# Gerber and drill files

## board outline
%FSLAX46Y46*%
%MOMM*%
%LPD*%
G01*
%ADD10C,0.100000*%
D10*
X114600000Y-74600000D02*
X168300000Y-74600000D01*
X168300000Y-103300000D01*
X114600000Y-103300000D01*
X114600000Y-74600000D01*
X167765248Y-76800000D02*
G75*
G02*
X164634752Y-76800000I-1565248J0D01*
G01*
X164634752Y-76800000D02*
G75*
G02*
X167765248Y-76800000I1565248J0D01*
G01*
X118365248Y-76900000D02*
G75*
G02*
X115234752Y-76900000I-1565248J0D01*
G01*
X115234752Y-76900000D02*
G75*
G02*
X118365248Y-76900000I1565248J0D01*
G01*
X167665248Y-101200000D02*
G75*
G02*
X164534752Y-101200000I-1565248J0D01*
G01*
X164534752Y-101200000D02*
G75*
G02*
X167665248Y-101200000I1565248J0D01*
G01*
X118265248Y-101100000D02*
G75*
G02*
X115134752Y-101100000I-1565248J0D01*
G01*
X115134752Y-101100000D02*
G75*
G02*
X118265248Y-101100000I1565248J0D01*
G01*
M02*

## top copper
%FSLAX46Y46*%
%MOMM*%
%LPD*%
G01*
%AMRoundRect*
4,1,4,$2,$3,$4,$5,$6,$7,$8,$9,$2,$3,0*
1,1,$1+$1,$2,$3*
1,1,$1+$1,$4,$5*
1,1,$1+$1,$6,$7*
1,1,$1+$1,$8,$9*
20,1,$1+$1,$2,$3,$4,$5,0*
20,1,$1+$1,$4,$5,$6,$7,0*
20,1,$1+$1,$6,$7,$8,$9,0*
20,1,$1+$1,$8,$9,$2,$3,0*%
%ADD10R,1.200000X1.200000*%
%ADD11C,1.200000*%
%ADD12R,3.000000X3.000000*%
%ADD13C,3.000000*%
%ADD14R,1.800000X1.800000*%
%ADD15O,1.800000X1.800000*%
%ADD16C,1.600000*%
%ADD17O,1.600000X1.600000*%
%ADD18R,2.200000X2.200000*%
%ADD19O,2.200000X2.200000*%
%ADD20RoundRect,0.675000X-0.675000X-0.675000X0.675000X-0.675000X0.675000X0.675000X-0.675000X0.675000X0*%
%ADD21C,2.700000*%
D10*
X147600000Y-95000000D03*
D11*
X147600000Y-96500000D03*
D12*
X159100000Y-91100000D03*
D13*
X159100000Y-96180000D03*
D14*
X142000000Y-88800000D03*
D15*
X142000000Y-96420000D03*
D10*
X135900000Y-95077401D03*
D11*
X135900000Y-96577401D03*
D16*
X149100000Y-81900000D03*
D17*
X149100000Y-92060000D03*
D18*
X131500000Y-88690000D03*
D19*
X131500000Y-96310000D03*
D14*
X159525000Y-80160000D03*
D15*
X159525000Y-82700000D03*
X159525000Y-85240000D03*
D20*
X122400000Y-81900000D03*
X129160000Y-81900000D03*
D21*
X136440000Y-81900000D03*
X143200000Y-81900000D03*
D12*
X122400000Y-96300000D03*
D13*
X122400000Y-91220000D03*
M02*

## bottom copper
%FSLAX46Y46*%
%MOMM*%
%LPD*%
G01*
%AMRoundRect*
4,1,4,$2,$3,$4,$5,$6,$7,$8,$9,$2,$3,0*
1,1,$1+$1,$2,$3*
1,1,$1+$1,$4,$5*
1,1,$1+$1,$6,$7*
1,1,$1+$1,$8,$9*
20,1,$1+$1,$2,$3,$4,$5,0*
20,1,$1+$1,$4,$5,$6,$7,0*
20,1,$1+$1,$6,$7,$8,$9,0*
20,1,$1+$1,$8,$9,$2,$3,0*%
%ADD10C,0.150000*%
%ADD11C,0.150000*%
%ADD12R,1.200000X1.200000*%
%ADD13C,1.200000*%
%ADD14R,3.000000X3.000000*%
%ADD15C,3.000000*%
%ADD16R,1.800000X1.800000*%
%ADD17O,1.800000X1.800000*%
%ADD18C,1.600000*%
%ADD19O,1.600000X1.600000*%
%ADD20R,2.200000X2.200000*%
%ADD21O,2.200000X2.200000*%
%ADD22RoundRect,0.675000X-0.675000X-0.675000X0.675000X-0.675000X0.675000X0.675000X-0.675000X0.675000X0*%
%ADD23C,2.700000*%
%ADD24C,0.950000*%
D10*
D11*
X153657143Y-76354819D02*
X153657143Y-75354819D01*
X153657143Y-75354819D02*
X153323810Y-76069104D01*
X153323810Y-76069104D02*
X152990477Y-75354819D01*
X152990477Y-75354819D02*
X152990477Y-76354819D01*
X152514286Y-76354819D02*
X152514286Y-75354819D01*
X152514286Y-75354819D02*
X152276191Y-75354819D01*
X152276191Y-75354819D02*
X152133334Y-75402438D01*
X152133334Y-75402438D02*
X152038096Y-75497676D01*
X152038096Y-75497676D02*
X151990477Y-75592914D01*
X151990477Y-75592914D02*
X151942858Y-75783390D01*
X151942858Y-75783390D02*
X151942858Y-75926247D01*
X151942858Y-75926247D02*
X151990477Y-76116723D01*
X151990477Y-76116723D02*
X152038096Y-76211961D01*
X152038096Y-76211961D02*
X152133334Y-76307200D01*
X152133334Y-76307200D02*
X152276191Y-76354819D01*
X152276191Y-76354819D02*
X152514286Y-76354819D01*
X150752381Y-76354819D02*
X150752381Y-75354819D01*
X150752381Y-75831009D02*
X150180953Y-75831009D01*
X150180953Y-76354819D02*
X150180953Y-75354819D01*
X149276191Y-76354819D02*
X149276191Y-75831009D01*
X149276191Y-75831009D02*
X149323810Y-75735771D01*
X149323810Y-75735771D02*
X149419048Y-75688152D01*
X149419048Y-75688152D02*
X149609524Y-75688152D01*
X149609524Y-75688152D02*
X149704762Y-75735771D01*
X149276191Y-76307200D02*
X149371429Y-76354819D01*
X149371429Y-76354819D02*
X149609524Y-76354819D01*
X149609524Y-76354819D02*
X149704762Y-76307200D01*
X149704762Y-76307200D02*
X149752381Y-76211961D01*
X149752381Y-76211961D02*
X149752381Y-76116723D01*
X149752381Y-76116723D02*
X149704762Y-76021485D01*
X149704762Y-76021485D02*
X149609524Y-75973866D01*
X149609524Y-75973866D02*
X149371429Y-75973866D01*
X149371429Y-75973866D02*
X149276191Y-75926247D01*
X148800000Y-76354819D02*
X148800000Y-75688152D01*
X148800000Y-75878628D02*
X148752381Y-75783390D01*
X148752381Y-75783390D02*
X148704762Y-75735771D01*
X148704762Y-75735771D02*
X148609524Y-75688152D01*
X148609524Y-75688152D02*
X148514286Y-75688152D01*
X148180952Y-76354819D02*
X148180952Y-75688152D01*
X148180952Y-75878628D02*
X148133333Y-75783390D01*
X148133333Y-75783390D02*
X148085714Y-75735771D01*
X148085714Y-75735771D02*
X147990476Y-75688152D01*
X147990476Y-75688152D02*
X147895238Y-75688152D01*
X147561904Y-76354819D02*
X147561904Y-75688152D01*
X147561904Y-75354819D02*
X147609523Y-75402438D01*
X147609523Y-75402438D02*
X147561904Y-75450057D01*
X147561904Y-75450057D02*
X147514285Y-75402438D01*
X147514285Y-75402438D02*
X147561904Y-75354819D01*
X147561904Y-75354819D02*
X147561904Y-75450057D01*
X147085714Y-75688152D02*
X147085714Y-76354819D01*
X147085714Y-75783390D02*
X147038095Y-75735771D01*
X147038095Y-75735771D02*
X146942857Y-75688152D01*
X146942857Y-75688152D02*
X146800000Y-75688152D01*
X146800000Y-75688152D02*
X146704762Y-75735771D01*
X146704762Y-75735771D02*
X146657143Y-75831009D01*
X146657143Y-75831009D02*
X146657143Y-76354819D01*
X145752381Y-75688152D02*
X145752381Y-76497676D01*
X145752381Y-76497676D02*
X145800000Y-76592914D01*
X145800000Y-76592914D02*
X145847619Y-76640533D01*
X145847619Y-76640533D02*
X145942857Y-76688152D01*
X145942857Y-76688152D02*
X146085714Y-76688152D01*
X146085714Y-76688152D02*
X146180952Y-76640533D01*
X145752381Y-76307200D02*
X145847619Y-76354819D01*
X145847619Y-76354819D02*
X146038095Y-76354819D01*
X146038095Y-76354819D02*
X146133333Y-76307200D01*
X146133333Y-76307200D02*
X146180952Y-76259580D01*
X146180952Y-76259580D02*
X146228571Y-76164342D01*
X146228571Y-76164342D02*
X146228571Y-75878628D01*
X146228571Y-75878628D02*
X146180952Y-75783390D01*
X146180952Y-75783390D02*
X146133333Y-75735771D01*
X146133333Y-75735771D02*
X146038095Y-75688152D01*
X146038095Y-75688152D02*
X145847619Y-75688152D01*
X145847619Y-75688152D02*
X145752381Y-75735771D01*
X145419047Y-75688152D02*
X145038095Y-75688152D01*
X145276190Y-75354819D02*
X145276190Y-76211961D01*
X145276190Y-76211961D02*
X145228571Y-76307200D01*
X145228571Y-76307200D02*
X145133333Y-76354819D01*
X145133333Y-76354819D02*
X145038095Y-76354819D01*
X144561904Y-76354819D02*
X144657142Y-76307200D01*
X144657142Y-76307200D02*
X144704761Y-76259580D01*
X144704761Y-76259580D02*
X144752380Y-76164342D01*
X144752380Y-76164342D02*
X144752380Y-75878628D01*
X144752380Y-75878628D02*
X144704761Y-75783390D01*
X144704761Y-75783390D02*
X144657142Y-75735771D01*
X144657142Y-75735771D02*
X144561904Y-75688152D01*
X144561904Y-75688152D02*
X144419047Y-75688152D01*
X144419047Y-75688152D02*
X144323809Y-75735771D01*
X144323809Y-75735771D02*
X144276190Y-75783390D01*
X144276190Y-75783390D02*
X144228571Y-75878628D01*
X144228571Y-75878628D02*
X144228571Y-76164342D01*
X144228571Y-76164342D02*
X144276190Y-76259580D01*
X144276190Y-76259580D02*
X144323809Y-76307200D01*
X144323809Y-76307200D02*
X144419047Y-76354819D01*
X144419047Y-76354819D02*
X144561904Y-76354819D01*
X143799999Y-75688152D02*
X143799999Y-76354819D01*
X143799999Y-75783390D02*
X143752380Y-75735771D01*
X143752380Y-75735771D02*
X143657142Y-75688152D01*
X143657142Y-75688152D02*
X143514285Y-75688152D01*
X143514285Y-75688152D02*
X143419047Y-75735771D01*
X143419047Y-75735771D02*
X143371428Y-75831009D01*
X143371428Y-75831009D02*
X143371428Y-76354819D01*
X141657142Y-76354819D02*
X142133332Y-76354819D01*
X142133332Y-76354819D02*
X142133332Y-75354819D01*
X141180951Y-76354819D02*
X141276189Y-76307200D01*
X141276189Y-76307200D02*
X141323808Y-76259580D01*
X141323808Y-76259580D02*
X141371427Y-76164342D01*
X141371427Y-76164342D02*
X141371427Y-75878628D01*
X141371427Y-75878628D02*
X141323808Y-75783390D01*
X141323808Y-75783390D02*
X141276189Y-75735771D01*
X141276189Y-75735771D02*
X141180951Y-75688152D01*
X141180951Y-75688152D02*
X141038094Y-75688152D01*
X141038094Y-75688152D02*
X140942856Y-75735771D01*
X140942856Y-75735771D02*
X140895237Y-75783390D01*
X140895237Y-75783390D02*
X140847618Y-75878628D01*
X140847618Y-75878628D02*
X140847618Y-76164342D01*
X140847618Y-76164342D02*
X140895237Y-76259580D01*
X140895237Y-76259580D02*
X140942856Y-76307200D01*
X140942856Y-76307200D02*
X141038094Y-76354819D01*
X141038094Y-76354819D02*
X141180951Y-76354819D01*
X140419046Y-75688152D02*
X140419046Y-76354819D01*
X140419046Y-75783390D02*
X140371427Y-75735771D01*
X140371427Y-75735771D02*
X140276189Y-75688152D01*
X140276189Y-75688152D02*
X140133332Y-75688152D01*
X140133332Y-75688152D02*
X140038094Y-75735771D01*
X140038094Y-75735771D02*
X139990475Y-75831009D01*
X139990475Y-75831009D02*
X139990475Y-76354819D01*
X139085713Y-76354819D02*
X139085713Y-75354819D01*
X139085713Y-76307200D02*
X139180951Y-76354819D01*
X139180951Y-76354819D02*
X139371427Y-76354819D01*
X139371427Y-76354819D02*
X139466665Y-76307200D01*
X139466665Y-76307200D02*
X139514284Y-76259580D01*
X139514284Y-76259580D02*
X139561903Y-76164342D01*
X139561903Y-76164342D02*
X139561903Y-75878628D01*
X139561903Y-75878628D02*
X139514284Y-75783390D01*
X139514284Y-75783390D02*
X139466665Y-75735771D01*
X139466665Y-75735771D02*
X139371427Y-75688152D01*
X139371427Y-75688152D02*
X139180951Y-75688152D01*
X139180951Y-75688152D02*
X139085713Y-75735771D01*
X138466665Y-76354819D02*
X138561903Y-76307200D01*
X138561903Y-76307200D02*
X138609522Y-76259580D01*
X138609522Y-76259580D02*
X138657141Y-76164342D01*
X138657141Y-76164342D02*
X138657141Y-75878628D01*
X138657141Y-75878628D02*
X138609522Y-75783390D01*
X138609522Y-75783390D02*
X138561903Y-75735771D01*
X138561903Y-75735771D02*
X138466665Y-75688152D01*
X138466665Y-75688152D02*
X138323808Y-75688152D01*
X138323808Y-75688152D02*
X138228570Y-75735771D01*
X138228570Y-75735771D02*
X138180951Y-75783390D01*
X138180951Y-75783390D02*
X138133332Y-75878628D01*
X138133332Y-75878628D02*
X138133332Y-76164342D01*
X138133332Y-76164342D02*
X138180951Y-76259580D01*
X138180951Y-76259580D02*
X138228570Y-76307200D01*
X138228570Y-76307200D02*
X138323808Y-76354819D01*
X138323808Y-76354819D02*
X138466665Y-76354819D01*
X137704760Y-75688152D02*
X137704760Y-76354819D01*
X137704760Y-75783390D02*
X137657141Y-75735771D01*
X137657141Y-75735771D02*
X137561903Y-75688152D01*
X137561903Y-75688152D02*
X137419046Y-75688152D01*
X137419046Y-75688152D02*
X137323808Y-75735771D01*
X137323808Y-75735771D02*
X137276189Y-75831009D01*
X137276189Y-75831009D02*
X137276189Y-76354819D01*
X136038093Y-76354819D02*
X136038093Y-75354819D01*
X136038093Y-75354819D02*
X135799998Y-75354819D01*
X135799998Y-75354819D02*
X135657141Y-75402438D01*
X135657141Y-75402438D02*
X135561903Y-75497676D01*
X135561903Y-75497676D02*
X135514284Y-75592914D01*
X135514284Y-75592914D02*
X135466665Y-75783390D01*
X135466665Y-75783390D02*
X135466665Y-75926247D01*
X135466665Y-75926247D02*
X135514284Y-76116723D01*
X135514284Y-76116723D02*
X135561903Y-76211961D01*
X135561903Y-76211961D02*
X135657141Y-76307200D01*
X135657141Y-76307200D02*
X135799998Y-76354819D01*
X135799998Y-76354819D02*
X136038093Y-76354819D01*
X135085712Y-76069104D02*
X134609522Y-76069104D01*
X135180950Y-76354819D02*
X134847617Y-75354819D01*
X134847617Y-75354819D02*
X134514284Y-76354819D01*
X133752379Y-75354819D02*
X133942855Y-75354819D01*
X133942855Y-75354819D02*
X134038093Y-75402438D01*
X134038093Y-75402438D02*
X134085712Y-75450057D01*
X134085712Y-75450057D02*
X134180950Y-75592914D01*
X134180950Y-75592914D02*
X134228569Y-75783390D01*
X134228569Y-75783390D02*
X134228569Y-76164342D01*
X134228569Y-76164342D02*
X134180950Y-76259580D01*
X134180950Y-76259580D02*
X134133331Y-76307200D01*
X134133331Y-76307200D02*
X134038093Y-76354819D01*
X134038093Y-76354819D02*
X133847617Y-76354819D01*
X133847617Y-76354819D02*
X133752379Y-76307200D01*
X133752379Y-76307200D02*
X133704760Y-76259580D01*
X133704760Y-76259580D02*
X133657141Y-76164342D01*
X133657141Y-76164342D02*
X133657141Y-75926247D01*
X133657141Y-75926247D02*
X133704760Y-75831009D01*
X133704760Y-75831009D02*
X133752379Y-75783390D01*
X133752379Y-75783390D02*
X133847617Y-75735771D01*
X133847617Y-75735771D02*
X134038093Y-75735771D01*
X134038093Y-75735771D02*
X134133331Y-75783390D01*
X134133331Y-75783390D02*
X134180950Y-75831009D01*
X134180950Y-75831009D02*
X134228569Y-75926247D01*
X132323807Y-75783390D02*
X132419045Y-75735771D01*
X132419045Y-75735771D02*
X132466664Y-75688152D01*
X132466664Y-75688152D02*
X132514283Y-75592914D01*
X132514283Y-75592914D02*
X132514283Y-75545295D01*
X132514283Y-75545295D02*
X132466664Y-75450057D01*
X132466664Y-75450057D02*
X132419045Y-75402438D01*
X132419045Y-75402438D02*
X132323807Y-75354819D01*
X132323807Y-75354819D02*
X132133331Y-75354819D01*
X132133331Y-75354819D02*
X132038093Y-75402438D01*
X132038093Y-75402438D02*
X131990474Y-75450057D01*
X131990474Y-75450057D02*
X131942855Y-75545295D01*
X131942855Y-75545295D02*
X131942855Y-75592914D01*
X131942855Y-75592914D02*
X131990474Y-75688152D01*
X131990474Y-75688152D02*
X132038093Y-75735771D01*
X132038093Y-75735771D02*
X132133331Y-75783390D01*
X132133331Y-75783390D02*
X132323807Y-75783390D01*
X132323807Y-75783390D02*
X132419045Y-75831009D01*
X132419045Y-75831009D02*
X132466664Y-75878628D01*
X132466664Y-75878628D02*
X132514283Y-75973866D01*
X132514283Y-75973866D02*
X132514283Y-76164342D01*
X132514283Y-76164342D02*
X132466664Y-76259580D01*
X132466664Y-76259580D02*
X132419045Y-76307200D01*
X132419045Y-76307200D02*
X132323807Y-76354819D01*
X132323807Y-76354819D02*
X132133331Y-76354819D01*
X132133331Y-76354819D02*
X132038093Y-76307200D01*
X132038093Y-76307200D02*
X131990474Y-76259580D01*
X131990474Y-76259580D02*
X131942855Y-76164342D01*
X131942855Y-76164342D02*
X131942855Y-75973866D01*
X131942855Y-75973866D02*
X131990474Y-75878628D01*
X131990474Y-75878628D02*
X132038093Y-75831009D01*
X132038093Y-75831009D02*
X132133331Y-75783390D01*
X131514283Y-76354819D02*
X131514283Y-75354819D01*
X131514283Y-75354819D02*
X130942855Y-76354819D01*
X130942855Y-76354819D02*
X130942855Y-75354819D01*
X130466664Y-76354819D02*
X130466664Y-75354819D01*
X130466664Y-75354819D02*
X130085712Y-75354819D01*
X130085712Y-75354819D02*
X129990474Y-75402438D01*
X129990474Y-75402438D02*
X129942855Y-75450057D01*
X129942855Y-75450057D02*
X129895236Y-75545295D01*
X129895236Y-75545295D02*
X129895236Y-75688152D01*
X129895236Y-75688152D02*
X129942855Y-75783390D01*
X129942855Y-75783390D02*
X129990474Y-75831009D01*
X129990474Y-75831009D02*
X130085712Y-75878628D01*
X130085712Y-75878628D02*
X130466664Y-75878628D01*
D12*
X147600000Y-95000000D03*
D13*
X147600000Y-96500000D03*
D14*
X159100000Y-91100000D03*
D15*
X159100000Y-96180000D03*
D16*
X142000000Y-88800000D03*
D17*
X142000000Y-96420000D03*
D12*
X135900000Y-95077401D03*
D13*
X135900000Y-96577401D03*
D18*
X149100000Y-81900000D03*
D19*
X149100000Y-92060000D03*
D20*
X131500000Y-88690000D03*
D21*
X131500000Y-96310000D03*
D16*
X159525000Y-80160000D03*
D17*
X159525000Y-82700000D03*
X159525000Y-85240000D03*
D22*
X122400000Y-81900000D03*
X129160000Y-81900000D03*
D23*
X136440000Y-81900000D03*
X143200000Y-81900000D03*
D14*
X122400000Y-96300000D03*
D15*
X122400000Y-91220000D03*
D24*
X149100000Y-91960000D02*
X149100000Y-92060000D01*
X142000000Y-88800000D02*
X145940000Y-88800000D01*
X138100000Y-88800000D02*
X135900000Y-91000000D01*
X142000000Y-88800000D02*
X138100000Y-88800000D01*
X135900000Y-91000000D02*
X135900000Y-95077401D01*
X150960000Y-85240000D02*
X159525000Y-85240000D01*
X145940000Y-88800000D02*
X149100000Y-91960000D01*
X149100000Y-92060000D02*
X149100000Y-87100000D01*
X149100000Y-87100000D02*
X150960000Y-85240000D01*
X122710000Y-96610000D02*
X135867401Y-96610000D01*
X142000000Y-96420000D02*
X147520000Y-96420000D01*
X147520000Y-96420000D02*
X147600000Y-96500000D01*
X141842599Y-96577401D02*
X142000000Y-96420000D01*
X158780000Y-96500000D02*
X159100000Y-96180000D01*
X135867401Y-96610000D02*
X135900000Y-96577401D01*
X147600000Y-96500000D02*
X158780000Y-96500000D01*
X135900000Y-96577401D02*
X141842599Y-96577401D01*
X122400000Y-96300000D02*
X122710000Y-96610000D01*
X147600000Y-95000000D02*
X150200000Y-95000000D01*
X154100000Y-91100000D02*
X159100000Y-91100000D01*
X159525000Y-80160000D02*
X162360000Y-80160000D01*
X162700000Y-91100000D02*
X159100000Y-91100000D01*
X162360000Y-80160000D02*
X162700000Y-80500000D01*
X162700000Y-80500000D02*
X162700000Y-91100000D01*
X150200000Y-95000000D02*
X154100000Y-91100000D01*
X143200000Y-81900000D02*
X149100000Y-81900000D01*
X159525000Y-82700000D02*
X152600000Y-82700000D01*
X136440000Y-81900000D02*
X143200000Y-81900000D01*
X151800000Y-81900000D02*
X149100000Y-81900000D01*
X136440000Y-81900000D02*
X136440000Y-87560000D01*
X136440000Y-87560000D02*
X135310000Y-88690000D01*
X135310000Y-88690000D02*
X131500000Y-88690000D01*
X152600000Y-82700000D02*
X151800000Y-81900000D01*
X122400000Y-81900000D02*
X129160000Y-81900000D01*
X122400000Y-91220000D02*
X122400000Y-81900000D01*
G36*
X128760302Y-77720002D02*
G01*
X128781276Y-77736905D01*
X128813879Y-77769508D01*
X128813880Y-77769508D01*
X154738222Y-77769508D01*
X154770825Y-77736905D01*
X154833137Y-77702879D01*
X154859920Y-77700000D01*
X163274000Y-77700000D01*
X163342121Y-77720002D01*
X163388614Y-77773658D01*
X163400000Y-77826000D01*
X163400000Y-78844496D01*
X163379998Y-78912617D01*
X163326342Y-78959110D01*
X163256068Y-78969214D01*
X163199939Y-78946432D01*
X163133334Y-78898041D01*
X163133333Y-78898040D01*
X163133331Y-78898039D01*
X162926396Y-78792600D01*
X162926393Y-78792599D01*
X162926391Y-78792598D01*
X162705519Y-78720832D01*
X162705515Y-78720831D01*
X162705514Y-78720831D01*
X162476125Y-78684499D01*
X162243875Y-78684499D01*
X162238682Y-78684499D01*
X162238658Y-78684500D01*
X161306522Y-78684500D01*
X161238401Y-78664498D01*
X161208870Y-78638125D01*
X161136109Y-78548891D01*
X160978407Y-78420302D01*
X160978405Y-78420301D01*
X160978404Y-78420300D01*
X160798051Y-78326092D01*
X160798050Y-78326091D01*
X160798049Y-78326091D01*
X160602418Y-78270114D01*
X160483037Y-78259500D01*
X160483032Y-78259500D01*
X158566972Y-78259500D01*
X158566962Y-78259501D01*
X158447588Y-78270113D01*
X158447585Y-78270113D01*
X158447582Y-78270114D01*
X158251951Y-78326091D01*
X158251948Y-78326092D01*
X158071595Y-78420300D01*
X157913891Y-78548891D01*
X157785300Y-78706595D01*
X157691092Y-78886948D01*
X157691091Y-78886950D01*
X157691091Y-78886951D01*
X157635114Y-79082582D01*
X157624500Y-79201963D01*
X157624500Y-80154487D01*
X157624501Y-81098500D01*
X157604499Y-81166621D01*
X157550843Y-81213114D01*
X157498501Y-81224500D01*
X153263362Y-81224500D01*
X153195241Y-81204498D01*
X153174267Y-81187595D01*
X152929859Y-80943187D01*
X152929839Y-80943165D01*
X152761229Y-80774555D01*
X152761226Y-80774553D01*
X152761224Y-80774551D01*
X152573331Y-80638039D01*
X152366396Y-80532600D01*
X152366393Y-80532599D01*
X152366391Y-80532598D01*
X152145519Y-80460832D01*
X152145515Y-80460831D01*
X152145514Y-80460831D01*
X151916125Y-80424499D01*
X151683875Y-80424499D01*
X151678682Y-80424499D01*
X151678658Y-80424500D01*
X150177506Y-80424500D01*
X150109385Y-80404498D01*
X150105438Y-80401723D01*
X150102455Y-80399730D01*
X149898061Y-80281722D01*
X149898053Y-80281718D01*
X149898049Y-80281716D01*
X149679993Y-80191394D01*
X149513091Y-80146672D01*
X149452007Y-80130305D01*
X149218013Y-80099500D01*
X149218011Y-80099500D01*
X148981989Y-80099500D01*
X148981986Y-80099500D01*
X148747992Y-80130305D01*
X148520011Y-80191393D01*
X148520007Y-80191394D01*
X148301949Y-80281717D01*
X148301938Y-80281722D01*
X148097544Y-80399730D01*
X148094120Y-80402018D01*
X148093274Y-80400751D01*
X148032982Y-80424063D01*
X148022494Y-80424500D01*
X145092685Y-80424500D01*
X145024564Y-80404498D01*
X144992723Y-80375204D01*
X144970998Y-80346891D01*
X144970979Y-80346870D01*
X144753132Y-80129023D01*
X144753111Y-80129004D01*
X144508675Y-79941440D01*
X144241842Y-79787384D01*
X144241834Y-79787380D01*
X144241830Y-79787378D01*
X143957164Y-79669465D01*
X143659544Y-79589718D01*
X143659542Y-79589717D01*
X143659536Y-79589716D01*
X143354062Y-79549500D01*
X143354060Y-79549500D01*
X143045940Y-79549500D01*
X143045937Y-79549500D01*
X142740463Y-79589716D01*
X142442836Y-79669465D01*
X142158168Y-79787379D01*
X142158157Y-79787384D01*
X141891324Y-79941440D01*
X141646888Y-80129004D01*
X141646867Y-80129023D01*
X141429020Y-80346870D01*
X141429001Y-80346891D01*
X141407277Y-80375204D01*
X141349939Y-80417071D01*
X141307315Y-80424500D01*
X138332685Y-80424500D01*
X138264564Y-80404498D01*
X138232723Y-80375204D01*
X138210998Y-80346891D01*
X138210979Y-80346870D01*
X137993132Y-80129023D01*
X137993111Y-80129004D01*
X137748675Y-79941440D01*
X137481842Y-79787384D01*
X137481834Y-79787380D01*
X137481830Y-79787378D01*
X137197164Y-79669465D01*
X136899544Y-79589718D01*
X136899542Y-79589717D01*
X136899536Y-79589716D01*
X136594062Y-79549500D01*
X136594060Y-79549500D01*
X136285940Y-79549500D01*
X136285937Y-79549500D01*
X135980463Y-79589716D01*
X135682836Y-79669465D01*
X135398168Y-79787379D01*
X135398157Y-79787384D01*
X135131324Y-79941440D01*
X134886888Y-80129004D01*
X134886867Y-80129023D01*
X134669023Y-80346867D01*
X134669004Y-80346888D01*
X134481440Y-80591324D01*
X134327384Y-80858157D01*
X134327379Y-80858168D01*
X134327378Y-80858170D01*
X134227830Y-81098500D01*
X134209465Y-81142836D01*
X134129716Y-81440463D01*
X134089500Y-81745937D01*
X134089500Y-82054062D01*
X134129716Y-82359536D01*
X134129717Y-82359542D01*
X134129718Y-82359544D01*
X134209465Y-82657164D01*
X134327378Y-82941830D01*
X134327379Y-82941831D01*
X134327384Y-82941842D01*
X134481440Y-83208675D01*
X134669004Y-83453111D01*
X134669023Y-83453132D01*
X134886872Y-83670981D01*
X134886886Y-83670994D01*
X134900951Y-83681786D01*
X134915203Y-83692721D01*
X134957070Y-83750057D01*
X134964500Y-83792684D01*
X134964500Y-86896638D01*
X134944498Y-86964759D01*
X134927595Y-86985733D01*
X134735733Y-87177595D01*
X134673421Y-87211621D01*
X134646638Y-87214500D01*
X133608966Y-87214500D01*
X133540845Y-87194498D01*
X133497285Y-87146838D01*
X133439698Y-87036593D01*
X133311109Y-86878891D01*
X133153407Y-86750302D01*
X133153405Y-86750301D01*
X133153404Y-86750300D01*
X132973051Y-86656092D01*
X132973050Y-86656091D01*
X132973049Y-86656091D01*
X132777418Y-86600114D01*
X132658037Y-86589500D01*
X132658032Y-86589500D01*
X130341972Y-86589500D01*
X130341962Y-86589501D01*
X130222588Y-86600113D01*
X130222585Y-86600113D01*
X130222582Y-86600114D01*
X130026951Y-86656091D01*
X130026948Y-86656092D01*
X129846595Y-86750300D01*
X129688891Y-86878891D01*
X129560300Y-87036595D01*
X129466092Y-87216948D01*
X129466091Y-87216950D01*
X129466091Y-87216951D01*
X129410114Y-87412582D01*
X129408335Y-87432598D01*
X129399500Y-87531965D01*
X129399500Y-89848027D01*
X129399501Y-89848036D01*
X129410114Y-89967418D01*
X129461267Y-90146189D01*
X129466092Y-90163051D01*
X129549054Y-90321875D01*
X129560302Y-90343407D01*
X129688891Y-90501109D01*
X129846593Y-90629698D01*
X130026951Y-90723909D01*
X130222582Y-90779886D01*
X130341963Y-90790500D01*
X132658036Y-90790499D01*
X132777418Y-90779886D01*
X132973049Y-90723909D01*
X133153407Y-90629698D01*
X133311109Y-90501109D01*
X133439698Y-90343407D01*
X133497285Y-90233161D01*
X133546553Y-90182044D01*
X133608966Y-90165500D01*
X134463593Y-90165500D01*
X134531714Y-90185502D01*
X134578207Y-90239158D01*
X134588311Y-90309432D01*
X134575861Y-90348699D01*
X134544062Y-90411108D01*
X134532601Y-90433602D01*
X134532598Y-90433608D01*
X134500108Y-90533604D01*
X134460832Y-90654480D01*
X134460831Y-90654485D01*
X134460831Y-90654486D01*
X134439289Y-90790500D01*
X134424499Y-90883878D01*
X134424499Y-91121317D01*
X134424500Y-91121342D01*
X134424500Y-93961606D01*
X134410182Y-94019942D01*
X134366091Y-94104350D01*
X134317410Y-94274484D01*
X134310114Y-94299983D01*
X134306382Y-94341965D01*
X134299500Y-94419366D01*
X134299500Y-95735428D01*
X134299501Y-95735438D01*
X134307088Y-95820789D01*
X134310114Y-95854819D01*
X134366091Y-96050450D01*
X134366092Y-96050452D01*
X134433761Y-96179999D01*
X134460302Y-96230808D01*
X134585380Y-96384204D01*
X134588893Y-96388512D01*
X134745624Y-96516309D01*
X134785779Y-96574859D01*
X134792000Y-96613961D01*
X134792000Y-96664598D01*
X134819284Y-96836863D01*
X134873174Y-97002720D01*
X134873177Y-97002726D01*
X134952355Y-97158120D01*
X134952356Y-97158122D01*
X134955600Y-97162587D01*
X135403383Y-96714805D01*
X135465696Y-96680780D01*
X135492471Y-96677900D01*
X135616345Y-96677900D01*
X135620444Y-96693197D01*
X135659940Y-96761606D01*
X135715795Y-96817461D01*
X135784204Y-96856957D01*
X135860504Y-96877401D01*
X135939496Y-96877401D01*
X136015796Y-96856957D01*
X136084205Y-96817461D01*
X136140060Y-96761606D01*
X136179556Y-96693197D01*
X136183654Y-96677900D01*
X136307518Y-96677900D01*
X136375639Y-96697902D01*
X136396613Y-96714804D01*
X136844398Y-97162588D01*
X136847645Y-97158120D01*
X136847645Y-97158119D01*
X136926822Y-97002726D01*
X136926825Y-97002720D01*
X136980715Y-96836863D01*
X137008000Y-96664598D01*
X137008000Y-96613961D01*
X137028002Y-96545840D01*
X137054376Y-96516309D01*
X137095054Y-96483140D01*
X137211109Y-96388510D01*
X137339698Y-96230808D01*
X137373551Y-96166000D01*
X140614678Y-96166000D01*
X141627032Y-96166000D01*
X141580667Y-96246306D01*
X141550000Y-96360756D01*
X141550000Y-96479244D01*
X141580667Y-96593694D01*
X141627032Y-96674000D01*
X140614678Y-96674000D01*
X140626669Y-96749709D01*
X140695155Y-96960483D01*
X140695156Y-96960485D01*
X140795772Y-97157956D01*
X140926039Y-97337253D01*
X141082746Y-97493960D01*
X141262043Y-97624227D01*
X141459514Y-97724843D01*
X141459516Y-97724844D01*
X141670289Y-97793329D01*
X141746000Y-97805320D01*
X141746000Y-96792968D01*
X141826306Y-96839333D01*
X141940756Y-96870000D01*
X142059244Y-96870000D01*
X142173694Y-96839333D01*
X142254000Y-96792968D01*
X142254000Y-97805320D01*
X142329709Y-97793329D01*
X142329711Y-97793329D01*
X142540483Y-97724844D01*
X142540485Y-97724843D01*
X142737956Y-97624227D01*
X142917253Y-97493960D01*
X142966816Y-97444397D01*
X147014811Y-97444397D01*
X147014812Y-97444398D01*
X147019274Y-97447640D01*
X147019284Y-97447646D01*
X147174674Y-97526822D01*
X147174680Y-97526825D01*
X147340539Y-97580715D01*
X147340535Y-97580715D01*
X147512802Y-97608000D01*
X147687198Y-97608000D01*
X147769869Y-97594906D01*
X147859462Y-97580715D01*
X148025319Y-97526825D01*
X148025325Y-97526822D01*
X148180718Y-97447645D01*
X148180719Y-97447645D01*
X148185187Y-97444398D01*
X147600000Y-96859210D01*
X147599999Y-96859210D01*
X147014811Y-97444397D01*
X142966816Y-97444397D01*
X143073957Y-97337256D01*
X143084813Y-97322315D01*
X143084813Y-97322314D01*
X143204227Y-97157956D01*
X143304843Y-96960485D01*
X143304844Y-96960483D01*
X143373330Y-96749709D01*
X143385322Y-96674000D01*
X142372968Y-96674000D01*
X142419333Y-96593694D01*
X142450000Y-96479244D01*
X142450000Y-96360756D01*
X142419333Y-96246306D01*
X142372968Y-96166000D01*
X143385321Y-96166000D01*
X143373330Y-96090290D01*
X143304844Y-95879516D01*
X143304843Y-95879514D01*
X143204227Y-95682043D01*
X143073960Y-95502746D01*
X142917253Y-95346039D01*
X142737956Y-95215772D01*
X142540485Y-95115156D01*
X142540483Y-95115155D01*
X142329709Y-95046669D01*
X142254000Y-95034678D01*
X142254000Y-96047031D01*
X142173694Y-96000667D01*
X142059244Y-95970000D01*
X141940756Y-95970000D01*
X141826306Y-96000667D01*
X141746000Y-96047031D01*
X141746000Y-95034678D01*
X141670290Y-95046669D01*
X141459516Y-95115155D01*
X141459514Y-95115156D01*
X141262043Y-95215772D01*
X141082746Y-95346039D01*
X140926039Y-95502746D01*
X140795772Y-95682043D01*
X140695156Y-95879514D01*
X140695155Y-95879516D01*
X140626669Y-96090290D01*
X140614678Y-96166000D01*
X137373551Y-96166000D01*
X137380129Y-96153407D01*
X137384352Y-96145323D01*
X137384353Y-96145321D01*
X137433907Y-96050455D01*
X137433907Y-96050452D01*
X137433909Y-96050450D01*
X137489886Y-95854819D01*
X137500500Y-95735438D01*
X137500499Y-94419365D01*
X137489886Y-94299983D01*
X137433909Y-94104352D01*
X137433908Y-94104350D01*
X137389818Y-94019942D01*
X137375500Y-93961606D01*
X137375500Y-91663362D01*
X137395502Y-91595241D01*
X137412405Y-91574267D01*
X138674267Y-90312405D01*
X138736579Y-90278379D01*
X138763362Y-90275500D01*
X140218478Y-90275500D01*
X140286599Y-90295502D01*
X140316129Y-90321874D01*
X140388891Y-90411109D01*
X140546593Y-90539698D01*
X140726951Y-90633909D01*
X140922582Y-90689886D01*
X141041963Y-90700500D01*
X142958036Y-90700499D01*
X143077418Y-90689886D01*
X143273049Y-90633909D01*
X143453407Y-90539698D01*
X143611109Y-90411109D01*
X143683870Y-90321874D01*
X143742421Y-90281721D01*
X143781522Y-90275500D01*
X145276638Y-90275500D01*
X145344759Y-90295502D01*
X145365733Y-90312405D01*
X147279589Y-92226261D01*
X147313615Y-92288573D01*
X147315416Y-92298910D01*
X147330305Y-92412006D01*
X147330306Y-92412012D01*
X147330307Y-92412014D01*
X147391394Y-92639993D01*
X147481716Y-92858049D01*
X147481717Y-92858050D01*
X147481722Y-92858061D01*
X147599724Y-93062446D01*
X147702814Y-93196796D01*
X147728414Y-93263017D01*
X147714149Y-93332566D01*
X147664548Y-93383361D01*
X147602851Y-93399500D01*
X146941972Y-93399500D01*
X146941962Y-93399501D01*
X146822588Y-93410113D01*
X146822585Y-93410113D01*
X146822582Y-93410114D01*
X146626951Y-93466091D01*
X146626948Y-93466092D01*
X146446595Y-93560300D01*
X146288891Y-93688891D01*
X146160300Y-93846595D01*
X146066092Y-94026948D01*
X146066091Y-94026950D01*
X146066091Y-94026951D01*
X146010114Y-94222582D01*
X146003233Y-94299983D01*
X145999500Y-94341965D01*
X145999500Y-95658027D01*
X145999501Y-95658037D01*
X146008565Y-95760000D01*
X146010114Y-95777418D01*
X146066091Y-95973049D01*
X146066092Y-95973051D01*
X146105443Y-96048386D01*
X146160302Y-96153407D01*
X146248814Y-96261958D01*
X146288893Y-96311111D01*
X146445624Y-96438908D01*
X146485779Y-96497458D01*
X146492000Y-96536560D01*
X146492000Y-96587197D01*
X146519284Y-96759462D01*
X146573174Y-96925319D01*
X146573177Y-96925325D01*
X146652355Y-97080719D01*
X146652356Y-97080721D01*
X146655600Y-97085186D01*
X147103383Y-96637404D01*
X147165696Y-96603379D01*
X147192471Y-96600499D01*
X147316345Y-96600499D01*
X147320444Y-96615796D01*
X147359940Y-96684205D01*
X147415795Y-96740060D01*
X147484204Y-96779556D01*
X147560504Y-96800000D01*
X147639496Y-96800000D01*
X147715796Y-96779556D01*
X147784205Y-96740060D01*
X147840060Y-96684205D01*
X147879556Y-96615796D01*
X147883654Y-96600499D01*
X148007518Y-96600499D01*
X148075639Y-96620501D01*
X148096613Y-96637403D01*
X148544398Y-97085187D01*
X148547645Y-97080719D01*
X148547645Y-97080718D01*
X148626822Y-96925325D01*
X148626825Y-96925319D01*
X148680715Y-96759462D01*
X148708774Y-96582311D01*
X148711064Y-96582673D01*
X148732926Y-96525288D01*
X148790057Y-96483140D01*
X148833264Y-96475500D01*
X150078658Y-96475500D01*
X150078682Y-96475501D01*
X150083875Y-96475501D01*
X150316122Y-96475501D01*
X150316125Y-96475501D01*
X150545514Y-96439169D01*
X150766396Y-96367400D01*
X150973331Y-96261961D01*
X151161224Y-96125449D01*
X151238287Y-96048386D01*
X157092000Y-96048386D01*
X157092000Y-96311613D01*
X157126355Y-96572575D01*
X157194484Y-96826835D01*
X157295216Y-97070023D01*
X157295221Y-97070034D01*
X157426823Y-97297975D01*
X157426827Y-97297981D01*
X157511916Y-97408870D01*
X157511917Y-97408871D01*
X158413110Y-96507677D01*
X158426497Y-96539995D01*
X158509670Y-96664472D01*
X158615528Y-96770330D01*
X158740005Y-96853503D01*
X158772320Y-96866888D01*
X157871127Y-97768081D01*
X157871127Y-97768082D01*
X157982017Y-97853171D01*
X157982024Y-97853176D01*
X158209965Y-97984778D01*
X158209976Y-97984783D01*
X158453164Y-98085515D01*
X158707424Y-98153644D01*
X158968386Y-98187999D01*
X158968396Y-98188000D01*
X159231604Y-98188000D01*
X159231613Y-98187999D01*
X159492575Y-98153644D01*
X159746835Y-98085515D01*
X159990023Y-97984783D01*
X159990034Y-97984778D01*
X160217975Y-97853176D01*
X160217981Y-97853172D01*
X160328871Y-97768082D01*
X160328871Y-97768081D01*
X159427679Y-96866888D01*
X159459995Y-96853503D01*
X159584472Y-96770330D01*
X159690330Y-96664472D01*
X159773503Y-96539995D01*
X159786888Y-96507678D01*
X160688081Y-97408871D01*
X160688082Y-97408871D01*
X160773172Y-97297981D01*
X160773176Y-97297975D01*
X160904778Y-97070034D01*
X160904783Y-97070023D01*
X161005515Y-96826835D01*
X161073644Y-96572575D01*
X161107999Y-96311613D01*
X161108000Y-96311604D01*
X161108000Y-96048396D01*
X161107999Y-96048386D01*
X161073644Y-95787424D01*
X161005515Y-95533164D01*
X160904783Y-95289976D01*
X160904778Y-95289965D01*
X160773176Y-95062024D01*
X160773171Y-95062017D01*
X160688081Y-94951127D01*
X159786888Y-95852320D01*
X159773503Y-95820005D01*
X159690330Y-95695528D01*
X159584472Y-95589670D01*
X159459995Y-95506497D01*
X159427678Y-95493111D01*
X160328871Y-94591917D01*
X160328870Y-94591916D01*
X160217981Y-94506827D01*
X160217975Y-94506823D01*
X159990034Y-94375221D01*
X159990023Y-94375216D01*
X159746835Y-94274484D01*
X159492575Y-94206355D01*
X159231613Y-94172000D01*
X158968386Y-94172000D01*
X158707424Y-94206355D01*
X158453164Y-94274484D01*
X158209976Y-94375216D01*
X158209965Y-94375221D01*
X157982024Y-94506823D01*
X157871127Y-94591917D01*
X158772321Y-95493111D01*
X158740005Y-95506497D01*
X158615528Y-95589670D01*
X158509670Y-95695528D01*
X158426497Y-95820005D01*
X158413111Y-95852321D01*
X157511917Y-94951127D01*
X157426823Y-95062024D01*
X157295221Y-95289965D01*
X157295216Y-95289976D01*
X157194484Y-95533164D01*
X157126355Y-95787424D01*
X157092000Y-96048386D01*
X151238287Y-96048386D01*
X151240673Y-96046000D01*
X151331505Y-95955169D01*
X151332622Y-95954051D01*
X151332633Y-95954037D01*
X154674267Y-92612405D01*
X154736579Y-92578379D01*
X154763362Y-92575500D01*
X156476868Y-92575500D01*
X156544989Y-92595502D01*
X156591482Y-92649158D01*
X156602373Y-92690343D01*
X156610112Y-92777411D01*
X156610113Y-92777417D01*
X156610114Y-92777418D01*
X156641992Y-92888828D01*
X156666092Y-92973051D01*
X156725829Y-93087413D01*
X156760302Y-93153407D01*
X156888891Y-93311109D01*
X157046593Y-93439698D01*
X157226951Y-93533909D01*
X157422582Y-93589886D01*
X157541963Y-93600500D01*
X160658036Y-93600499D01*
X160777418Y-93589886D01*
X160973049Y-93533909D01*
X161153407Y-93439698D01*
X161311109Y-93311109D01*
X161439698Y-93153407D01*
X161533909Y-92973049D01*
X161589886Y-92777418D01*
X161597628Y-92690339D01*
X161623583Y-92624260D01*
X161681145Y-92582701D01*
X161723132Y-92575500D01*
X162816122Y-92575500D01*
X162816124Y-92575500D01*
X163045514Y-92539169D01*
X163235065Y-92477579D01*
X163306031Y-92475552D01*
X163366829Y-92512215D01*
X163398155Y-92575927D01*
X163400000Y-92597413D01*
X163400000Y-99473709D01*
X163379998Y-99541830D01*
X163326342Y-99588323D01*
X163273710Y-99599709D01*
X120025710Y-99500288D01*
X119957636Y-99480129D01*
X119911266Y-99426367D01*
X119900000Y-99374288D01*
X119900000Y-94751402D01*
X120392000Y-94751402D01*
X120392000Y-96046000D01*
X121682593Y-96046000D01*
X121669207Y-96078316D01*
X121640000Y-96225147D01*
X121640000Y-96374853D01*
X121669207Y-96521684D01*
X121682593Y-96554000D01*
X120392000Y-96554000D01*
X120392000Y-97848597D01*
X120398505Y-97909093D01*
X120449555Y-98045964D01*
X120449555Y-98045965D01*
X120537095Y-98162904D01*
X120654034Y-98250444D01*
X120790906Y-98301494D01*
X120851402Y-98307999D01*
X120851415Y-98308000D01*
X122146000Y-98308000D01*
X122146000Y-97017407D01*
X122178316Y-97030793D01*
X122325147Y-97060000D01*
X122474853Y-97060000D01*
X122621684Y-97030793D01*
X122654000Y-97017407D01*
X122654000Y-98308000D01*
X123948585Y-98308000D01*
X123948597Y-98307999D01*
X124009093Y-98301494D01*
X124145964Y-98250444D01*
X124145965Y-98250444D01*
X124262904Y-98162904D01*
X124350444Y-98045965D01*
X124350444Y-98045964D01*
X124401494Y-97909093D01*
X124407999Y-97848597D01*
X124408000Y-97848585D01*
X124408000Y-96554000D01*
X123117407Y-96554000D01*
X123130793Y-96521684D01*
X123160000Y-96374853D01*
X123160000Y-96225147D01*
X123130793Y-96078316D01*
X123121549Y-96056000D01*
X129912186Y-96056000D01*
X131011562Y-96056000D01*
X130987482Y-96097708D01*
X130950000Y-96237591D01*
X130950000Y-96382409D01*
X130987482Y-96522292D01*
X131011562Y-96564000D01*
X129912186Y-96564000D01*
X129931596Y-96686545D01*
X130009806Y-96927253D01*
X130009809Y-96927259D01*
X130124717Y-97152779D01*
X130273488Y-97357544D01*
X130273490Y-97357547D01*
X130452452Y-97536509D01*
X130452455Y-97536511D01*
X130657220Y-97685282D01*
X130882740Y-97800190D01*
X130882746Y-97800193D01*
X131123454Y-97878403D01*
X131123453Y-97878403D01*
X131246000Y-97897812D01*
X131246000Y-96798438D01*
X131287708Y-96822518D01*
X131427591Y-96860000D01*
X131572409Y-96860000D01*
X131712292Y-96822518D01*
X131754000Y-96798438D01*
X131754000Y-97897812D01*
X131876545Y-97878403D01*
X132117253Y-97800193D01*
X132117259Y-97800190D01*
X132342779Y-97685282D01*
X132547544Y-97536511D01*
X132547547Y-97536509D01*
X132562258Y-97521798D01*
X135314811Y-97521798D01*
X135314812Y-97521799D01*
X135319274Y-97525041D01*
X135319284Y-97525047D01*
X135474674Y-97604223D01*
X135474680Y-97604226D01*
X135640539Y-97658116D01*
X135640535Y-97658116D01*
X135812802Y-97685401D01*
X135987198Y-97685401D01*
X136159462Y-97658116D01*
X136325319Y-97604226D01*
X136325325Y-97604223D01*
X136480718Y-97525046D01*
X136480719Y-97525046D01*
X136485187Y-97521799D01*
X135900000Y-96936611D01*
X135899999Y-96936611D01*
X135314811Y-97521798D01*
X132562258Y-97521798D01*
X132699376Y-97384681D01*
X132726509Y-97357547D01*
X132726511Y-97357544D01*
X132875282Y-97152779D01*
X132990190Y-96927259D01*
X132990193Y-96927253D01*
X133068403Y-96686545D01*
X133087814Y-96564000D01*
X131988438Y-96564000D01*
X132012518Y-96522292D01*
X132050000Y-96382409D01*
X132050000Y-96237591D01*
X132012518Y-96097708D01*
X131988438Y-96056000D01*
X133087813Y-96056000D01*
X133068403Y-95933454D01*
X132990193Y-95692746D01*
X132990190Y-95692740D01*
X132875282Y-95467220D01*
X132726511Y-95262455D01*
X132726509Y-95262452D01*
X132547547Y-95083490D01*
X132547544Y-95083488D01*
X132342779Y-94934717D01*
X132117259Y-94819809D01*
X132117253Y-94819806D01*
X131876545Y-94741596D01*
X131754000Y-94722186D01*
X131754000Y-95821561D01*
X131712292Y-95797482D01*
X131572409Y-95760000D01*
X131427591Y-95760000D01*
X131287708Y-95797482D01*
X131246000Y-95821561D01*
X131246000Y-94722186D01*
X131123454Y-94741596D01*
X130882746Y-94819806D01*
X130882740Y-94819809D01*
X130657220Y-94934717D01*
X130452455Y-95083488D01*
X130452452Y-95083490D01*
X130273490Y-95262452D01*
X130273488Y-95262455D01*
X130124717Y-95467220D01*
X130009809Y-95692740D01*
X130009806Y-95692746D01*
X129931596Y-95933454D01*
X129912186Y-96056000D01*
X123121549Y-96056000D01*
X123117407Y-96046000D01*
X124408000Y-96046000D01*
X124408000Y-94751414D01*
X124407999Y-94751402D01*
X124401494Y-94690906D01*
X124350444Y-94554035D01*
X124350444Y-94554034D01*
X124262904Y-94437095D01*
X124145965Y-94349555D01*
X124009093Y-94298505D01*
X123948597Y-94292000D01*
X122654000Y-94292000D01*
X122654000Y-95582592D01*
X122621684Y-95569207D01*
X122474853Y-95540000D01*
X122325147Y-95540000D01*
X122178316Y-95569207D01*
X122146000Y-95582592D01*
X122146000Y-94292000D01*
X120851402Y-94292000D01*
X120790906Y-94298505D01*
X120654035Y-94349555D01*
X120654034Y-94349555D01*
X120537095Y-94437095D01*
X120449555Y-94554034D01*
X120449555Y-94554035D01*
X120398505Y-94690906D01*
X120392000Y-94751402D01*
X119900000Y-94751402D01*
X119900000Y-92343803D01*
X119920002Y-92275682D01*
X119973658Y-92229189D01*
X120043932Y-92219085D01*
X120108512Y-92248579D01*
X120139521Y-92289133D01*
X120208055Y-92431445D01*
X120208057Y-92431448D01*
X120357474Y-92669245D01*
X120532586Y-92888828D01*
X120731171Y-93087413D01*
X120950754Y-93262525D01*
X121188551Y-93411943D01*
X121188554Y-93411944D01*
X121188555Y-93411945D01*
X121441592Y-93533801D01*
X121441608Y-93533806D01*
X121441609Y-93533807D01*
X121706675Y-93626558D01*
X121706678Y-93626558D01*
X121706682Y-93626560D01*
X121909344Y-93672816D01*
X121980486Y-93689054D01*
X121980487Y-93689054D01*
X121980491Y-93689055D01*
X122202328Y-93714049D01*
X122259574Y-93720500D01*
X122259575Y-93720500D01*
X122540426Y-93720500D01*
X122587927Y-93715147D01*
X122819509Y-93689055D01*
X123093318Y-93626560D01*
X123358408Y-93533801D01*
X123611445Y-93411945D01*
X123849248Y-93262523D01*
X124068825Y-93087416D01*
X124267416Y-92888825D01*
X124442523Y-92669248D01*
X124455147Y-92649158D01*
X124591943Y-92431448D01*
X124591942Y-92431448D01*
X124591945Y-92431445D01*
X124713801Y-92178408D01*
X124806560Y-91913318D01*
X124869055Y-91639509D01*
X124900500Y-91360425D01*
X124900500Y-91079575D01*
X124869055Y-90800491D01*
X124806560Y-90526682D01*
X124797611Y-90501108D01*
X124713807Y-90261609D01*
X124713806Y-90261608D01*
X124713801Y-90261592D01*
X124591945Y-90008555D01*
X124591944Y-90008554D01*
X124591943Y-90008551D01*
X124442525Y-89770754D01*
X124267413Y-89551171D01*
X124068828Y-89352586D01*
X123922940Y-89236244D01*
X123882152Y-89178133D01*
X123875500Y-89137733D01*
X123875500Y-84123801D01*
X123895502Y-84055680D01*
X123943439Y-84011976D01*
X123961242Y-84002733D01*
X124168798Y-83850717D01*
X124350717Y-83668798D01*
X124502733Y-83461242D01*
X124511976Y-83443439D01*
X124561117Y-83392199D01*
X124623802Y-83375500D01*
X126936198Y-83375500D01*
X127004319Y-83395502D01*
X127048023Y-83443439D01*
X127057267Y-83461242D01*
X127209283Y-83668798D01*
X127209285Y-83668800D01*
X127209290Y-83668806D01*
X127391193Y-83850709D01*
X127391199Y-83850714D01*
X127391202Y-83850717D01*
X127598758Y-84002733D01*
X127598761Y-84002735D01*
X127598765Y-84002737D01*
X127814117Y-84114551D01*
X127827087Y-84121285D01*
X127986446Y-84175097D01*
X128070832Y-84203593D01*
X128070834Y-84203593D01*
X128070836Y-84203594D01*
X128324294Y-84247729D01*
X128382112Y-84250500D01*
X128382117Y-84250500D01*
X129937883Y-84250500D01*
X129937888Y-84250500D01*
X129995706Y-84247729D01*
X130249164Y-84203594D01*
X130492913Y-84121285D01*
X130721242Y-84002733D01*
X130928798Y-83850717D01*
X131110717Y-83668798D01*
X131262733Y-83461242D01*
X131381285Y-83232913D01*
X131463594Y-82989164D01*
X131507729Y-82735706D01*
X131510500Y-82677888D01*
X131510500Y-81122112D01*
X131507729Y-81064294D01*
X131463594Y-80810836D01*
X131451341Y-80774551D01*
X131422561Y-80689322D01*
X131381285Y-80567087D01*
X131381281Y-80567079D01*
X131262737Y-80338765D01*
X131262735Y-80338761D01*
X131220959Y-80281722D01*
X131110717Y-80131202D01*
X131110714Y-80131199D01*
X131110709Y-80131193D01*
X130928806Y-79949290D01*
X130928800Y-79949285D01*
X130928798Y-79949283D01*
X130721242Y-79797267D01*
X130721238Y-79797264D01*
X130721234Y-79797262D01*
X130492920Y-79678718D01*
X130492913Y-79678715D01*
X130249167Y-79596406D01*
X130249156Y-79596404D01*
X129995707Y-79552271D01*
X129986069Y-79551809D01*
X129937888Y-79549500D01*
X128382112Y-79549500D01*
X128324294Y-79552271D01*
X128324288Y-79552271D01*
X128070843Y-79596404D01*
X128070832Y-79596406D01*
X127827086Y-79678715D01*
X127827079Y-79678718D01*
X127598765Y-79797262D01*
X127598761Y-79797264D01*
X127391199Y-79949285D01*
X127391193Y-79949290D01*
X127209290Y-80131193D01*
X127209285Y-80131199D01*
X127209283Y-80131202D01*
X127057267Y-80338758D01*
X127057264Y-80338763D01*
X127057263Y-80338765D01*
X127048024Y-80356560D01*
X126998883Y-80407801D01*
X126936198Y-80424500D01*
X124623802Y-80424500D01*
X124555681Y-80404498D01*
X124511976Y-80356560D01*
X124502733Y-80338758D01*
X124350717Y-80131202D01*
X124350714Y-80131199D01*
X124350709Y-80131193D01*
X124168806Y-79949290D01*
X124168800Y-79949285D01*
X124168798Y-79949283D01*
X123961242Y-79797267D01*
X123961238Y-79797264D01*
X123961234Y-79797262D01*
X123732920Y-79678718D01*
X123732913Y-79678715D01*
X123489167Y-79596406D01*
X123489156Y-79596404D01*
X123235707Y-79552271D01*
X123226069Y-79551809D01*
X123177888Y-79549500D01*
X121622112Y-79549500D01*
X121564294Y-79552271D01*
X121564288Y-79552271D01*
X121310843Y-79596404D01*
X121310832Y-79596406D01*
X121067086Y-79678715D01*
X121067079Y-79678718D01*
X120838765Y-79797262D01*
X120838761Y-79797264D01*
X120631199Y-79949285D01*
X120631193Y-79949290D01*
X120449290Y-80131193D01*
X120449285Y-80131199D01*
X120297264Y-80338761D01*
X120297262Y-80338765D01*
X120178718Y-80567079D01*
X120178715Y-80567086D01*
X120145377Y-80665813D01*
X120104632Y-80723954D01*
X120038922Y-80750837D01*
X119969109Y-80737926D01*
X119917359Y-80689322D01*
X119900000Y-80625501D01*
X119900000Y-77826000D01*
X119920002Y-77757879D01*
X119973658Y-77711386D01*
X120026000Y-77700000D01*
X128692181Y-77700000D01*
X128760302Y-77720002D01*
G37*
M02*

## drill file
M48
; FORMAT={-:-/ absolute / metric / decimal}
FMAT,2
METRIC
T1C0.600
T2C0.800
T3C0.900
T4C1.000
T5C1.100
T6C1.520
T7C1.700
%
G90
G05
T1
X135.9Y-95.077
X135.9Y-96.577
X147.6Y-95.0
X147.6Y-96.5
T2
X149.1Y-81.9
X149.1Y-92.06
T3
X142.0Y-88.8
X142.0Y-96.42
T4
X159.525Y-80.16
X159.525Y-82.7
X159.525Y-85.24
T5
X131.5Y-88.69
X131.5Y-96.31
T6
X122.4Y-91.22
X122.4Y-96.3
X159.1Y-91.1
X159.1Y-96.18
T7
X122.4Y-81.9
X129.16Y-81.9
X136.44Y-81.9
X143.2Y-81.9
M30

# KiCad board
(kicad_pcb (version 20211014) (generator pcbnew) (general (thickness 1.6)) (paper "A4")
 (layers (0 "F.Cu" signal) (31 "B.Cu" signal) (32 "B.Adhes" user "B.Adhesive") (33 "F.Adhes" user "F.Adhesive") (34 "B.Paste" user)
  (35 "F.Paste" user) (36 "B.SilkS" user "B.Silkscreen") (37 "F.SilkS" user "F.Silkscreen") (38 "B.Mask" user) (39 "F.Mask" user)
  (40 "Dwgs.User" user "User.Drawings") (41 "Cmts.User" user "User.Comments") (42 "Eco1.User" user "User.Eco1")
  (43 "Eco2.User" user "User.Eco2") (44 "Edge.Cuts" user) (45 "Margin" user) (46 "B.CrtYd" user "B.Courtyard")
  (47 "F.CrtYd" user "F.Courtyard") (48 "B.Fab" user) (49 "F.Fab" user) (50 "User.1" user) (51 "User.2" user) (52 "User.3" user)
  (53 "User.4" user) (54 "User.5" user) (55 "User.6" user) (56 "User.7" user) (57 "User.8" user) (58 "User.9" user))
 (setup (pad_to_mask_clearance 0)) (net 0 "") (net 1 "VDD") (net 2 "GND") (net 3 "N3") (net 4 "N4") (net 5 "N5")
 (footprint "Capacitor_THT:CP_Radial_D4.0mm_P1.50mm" (layer "F.Cu") (at 147.6 95 -90)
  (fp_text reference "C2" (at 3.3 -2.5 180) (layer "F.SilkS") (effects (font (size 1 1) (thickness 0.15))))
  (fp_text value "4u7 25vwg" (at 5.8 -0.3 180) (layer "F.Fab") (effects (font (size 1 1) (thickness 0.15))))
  (pad "1" thru_hole rect (at 0 0 270) (size 1.2 1.2) (drill 0.6) (layers *.Cu *.Mask) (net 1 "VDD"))
  (pad "2" thru_hole circle (at 1.5 0 270) (size 1.2 1.2) (drill 0.6) (layers *.Cu *.Mask) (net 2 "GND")))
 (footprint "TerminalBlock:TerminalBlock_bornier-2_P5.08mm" (layer "F.Cu") (at 159.1 91.1 -90)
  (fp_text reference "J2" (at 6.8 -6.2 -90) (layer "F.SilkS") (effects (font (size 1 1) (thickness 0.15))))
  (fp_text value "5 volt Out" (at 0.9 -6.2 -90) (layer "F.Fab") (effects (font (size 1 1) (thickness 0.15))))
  (pad "1" thru_hole rect (at 0 0 270) (size 3 3) (drill 1.52) (layers *.Cu *.Mask) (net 1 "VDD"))
  (pad "2" thru_hole circle (at 5.08 0 270) (size 3 3) (drill 1.52) (layers *.Cu *.Mask) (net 2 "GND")))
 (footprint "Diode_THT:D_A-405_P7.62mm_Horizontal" (layer "F.Cu") (at 142 88.8 -90)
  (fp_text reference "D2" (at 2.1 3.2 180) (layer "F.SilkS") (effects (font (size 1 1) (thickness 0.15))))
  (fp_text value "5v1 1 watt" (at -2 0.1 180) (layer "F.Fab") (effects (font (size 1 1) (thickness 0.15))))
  (pad "1" thru_hole rect (at 0 0 270) (size 1.8 1.8) (drill 0.9) (layers *.Cu *.Mask) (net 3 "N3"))
  (pad "2" thru_hole oval (at 7.62 0 270) (size 1.8 1.8) (drill 0.9) (layers *.Cu *.Mask) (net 2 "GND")))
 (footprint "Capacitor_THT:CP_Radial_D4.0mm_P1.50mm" (layer "F.Cu") (at 135.9 95.077401 -90)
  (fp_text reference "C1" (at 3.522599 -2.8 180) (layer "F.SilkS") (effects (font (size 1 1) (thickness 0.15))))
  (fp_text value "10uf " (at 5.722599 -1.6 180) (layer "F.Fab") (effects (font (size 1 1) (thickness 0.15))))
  (pad "1" thru_hole rect (at 0 0 270) (size 1.2 1.2) (drill 0.6) (layers *.Cu *.Mask) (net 3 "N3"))
  (pad "2" thru_hole circle (at 1.5 0 270) (size 1.2 1.2) (drill 0.6) (layers *.Cu *.Mask) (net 2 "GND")))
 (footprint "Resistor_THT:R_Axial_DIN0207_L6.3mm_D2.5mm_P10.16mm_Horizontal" (layer "F.Cu") (at 149.1 81.9 -90)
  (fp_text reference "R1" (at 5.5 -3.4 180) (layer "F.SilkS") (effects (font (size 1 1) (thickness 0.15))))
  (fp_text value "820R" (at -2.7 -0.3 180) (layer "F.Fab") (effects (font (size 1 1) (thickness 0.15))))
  (pad "1" thru_hole circle (at 0 0 270) (size 1.6 1.6) (drill 0.8) (layers *.Cu *.Mask) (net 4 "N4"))
  (pad "2" thru_hole oval (at 10.16 0 270) (size 1.6 1.6) (drill 0.8) (layers *.Cu *.Mask) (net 3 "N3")))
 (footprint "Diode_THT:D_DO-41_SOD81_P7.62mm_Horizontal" (layer "F.Cu") (at 131.5 88.69 -90)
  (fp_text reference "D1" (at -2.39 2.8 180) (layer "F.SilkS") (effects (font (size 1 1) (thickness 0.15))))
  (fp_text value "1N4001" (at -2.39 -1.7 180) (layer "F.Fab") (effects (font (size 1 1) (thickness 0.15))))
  (pad "1" thru_hole rect (at 0 0 270) (size 2.2 2.2) (drill 1.1) (layers *.Cu *.Mask) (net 4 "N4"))
  (pad "2" thru_hole oval (at 7.62 0 270) (size 2.2 2.2) (drill 1.1) (layers *.Cu *.Mask) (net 2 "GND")))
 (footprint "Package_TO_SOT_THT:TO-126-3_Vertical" (layer "F.Cu") (at 159.525 80.16 -90)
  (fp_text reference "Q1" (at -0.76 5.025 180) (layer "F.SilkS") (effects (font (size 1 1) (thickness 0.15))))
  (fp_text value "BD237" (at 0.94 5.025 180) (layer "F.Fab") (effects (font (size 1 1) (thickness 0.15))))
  (pad "1" thru_hole rect (at 0 0 270) (size 1.8 1.8) (drill 1) (layers *.Cu *.Mask) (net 1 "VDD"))
  (pad "2" thru_hole oval (at 2.54 0 270) (size 1.8 1.8) (drill 1) (layers *.Cu *.Mask) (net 4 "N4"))
  (pad "3" thru_hole oval (at 5.08 0 270) (size 1.8 1.8) (drill 1) (layers *.Cu *.Mask) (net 3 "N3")))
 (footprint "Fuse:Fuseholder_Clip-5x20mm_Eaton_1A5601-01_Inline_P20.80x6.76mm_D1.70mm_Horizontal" (layer "F.Cu") (at 122.4 81.9)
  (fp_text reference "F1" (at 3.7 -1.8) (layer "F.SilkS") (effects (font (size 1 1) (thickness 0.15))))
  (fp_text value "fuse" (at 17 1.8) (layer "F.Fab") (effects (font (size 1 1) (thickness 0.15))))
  (pad "1" thru_hole roundrect (at 0 0) (size 2.7 2.7) (drill 1.7) (layers *.Cu *.Mask) (roundrect_rratio 0.25) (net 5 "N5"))
  (pad "1" thru_hole roundrect (at 6.76 0) (size 2.7 2.7) (drill 1.7) (layers *.Cu *.Mask) (roundrect_rratio 0.25) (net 5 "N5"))
  (pad "2" thru_hole circle (at 14.04 0) (size 2.7 2.7) (drill 1.7) (layers *.Cu *.Mask) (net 4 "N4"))
  (pad "2" thru_hole circle (at 20.8 0) (size 2.7 2.7) (drill 1.7) (layers *.Cu *.Mask) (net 4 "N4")))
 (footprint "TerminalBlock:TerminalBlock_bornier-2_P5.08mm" (layer "F.Cu") (at 122.4 96.3 90)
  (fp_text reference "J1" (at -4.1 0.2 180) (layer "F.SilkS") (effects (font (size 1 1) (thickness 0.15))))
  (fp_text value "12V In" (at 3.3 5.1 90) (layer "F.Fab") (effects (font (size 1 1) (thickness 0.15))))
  (pad "1" thru_hole rect (at 0 0 90) (size 3 3) (drill 1.52) (layers *.Cu *.Mask) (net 2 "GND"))
  (pad "2" thru_hole circle (at 5.08 0 90) (size 3 3) (drill 1.52) (layers *.Cu *.Mask) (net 5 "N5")))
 (gr_rect (start 114.6 74.6) (end 168.3 103.3) (layer "Edge.Cuts") (width 0.1) (fill none))
 (gr_circle (center 166.2 76.8) (end 167.6 77.5) (layer "Edge.Cuts") (width 0.1) (fill none))
 (gr_circle (center 116.8 76.9) (end 118.2 77.6) (layer "Edge.Cuts") (width 0.1) (fill none))
 (gr_circle (center 166.1 101.2) (end 167.5 101.9) (layer "Edge.Cuts") (width 0.1) (fill none))
 (gr_circle (center 116.7 101.1) (end 118.1 101.8) (layer "Edge.Cuts") (width 0.1) (fill none))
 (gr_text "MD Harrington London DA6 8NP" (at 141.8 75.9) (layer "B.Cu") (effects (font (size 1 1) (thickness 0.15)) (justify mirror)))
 (segment (start 149.1 91.96) (end 149.1 92.06) (width 0.95) (layer "B.Cu") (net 3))
 (segment (start 142 88.8) (end 145.94 88.8) (width 0.95) (layer "B.Cu") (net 3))
 (segment (start 138.1 88.8) (end 135.9 91) (width 0.95) (layer "B.Cu") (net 3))
 (segment (start 142 88.8) (end 138.1 88.8) (width 0.95) (layer "B.Cu") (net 3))
 (segment (start 135.9 91) (end 135.9 95.077401) (width 0.95) (layer "B.Cu") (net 3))
 (segment (start 150.96 85.24) (end 159.525 85.24) (width 0.95) (layer "B.Cu") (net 3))
 (segment (start 145.94 88.8) (end 149.1 91.96) (width 0.95) (layer "B.Cu") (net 3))
 (segment (start 149.1 92.06) (end 149.1 87.1) (width 0.95) (layer "B.Cu") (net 3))
 (segment (start 149.1 87.1) (end 150.96 85.24) (width 0.95) (layer "B.Cu") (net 3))
 (segment (start 122.71 96.61) (end 135.867401 96.61) (width 0.95) (layer "B.Cu") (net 2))
 (segment (start 142 96.42) (end 147.52 96.42) (width 0.95) (layer "B.Cu") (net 2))
 (segment (start 147.52 96.42) (end 147.6 96.5) (width 0.95) (layer "B.Cu") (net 2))
 (segment (start 141.842599 96.577401) (end 142 96.42) (width 0.95) (layer "B.Cu") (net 2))
 (segment (start 158.78 96.5) (end 159.1 96.18) (width 0.95) (layer "B.Cu") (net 2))
 (segment (start 135.867401 96.61) (end 135.9 96.577401) (width 0.95) (layer "B.Cu") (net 2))
 (segment (start 147.6 96.5) (end 158.78 96.5) (width 0.95) (layer "B.Cu") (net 2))
 (segment (start 135.9 96.577401) (end 141.842599 96.577401) (width 0.95) (layer "B.Cu") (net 2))
 (segment (start 122.4 96.3) (end 122.71 96.61) (width 0.95) (layer "B.Cu") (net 2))
 (segment (start 147.6 95) (end 150.2 95) (width 0.95) (layer "B.Cu") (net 1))
 (segment (start 154.1 91.1) (end 159.1 91.1) (width 0.95) (layer "B.Cu") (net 1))
 (segment (start 159.525 80.16) (end 162.36 80.16) (width 0.95) (layer "B.Cu") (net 1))
 (segment (start 162.7 91.1) (end 159.1 91.1) (width 0.95) (layer "B.Cu") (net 1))
 (segment (start 162.36 80.16) (end 162.7 80.5) (width 0.95) (layer "B.Cu") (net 1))
 (segment (start 162.7 80.5) (end 162.7 91.1) (width 0.95) (layer "B.Cu") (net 1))
 (segment (start 150.2 95) (end 154.1 91.1) (width 0.95) (layer "B.Cu") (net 1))
 (segment (start 143.2 81.9) (end 149.1 81.9) (width 0.95) (layer "B.Cu") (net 4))
 (segment (start 159.525 82.7) (end 152.6 82.7) (width 0.95) (layer "B.Cu") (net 4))
 (segment (start 136.44 81.9) (end 143.2 81.9) (width 0.95) (layer "B.Cu") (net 4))
 (segment (start 151.8 81.9) (end 149.1 81.9) (width 0.95) (layer "B.Cu") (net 4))
 (segment (start 136.44 81.9) (end 136.44 87.56) (width 0.95) (layer "B.Cu") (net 4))
 (segment (start 136.44 87.56) (end 135.31 88.69) (width 0.95) (layer "B.Cu") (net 4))
 (segment (start 135.31 88.69) (end 131.5 88.69) (width 0.95) (layer "B.Cu") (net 4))
 (segment (start 152.6 82.7) (end 151.8 81.9) (width 0.95) (layer "B.Cu") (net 4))
 (segment (start 122.4 81.9) (end 129.16 81.9) (width 0.95) (layer "B.Cu") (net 5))
 (segment (start 122.4 91.22) (end 122.4 81.9) (width 0.95) (layer "B.Cu") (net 5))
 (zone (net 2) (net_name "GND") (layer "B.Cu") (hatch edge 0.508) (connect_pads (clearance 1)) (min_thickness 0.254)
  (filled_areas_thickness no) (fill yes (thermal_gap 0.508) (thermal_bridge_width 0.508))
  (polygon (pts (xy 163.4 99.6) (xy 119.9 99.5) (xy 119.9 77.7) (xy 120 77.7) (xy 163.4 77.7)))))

